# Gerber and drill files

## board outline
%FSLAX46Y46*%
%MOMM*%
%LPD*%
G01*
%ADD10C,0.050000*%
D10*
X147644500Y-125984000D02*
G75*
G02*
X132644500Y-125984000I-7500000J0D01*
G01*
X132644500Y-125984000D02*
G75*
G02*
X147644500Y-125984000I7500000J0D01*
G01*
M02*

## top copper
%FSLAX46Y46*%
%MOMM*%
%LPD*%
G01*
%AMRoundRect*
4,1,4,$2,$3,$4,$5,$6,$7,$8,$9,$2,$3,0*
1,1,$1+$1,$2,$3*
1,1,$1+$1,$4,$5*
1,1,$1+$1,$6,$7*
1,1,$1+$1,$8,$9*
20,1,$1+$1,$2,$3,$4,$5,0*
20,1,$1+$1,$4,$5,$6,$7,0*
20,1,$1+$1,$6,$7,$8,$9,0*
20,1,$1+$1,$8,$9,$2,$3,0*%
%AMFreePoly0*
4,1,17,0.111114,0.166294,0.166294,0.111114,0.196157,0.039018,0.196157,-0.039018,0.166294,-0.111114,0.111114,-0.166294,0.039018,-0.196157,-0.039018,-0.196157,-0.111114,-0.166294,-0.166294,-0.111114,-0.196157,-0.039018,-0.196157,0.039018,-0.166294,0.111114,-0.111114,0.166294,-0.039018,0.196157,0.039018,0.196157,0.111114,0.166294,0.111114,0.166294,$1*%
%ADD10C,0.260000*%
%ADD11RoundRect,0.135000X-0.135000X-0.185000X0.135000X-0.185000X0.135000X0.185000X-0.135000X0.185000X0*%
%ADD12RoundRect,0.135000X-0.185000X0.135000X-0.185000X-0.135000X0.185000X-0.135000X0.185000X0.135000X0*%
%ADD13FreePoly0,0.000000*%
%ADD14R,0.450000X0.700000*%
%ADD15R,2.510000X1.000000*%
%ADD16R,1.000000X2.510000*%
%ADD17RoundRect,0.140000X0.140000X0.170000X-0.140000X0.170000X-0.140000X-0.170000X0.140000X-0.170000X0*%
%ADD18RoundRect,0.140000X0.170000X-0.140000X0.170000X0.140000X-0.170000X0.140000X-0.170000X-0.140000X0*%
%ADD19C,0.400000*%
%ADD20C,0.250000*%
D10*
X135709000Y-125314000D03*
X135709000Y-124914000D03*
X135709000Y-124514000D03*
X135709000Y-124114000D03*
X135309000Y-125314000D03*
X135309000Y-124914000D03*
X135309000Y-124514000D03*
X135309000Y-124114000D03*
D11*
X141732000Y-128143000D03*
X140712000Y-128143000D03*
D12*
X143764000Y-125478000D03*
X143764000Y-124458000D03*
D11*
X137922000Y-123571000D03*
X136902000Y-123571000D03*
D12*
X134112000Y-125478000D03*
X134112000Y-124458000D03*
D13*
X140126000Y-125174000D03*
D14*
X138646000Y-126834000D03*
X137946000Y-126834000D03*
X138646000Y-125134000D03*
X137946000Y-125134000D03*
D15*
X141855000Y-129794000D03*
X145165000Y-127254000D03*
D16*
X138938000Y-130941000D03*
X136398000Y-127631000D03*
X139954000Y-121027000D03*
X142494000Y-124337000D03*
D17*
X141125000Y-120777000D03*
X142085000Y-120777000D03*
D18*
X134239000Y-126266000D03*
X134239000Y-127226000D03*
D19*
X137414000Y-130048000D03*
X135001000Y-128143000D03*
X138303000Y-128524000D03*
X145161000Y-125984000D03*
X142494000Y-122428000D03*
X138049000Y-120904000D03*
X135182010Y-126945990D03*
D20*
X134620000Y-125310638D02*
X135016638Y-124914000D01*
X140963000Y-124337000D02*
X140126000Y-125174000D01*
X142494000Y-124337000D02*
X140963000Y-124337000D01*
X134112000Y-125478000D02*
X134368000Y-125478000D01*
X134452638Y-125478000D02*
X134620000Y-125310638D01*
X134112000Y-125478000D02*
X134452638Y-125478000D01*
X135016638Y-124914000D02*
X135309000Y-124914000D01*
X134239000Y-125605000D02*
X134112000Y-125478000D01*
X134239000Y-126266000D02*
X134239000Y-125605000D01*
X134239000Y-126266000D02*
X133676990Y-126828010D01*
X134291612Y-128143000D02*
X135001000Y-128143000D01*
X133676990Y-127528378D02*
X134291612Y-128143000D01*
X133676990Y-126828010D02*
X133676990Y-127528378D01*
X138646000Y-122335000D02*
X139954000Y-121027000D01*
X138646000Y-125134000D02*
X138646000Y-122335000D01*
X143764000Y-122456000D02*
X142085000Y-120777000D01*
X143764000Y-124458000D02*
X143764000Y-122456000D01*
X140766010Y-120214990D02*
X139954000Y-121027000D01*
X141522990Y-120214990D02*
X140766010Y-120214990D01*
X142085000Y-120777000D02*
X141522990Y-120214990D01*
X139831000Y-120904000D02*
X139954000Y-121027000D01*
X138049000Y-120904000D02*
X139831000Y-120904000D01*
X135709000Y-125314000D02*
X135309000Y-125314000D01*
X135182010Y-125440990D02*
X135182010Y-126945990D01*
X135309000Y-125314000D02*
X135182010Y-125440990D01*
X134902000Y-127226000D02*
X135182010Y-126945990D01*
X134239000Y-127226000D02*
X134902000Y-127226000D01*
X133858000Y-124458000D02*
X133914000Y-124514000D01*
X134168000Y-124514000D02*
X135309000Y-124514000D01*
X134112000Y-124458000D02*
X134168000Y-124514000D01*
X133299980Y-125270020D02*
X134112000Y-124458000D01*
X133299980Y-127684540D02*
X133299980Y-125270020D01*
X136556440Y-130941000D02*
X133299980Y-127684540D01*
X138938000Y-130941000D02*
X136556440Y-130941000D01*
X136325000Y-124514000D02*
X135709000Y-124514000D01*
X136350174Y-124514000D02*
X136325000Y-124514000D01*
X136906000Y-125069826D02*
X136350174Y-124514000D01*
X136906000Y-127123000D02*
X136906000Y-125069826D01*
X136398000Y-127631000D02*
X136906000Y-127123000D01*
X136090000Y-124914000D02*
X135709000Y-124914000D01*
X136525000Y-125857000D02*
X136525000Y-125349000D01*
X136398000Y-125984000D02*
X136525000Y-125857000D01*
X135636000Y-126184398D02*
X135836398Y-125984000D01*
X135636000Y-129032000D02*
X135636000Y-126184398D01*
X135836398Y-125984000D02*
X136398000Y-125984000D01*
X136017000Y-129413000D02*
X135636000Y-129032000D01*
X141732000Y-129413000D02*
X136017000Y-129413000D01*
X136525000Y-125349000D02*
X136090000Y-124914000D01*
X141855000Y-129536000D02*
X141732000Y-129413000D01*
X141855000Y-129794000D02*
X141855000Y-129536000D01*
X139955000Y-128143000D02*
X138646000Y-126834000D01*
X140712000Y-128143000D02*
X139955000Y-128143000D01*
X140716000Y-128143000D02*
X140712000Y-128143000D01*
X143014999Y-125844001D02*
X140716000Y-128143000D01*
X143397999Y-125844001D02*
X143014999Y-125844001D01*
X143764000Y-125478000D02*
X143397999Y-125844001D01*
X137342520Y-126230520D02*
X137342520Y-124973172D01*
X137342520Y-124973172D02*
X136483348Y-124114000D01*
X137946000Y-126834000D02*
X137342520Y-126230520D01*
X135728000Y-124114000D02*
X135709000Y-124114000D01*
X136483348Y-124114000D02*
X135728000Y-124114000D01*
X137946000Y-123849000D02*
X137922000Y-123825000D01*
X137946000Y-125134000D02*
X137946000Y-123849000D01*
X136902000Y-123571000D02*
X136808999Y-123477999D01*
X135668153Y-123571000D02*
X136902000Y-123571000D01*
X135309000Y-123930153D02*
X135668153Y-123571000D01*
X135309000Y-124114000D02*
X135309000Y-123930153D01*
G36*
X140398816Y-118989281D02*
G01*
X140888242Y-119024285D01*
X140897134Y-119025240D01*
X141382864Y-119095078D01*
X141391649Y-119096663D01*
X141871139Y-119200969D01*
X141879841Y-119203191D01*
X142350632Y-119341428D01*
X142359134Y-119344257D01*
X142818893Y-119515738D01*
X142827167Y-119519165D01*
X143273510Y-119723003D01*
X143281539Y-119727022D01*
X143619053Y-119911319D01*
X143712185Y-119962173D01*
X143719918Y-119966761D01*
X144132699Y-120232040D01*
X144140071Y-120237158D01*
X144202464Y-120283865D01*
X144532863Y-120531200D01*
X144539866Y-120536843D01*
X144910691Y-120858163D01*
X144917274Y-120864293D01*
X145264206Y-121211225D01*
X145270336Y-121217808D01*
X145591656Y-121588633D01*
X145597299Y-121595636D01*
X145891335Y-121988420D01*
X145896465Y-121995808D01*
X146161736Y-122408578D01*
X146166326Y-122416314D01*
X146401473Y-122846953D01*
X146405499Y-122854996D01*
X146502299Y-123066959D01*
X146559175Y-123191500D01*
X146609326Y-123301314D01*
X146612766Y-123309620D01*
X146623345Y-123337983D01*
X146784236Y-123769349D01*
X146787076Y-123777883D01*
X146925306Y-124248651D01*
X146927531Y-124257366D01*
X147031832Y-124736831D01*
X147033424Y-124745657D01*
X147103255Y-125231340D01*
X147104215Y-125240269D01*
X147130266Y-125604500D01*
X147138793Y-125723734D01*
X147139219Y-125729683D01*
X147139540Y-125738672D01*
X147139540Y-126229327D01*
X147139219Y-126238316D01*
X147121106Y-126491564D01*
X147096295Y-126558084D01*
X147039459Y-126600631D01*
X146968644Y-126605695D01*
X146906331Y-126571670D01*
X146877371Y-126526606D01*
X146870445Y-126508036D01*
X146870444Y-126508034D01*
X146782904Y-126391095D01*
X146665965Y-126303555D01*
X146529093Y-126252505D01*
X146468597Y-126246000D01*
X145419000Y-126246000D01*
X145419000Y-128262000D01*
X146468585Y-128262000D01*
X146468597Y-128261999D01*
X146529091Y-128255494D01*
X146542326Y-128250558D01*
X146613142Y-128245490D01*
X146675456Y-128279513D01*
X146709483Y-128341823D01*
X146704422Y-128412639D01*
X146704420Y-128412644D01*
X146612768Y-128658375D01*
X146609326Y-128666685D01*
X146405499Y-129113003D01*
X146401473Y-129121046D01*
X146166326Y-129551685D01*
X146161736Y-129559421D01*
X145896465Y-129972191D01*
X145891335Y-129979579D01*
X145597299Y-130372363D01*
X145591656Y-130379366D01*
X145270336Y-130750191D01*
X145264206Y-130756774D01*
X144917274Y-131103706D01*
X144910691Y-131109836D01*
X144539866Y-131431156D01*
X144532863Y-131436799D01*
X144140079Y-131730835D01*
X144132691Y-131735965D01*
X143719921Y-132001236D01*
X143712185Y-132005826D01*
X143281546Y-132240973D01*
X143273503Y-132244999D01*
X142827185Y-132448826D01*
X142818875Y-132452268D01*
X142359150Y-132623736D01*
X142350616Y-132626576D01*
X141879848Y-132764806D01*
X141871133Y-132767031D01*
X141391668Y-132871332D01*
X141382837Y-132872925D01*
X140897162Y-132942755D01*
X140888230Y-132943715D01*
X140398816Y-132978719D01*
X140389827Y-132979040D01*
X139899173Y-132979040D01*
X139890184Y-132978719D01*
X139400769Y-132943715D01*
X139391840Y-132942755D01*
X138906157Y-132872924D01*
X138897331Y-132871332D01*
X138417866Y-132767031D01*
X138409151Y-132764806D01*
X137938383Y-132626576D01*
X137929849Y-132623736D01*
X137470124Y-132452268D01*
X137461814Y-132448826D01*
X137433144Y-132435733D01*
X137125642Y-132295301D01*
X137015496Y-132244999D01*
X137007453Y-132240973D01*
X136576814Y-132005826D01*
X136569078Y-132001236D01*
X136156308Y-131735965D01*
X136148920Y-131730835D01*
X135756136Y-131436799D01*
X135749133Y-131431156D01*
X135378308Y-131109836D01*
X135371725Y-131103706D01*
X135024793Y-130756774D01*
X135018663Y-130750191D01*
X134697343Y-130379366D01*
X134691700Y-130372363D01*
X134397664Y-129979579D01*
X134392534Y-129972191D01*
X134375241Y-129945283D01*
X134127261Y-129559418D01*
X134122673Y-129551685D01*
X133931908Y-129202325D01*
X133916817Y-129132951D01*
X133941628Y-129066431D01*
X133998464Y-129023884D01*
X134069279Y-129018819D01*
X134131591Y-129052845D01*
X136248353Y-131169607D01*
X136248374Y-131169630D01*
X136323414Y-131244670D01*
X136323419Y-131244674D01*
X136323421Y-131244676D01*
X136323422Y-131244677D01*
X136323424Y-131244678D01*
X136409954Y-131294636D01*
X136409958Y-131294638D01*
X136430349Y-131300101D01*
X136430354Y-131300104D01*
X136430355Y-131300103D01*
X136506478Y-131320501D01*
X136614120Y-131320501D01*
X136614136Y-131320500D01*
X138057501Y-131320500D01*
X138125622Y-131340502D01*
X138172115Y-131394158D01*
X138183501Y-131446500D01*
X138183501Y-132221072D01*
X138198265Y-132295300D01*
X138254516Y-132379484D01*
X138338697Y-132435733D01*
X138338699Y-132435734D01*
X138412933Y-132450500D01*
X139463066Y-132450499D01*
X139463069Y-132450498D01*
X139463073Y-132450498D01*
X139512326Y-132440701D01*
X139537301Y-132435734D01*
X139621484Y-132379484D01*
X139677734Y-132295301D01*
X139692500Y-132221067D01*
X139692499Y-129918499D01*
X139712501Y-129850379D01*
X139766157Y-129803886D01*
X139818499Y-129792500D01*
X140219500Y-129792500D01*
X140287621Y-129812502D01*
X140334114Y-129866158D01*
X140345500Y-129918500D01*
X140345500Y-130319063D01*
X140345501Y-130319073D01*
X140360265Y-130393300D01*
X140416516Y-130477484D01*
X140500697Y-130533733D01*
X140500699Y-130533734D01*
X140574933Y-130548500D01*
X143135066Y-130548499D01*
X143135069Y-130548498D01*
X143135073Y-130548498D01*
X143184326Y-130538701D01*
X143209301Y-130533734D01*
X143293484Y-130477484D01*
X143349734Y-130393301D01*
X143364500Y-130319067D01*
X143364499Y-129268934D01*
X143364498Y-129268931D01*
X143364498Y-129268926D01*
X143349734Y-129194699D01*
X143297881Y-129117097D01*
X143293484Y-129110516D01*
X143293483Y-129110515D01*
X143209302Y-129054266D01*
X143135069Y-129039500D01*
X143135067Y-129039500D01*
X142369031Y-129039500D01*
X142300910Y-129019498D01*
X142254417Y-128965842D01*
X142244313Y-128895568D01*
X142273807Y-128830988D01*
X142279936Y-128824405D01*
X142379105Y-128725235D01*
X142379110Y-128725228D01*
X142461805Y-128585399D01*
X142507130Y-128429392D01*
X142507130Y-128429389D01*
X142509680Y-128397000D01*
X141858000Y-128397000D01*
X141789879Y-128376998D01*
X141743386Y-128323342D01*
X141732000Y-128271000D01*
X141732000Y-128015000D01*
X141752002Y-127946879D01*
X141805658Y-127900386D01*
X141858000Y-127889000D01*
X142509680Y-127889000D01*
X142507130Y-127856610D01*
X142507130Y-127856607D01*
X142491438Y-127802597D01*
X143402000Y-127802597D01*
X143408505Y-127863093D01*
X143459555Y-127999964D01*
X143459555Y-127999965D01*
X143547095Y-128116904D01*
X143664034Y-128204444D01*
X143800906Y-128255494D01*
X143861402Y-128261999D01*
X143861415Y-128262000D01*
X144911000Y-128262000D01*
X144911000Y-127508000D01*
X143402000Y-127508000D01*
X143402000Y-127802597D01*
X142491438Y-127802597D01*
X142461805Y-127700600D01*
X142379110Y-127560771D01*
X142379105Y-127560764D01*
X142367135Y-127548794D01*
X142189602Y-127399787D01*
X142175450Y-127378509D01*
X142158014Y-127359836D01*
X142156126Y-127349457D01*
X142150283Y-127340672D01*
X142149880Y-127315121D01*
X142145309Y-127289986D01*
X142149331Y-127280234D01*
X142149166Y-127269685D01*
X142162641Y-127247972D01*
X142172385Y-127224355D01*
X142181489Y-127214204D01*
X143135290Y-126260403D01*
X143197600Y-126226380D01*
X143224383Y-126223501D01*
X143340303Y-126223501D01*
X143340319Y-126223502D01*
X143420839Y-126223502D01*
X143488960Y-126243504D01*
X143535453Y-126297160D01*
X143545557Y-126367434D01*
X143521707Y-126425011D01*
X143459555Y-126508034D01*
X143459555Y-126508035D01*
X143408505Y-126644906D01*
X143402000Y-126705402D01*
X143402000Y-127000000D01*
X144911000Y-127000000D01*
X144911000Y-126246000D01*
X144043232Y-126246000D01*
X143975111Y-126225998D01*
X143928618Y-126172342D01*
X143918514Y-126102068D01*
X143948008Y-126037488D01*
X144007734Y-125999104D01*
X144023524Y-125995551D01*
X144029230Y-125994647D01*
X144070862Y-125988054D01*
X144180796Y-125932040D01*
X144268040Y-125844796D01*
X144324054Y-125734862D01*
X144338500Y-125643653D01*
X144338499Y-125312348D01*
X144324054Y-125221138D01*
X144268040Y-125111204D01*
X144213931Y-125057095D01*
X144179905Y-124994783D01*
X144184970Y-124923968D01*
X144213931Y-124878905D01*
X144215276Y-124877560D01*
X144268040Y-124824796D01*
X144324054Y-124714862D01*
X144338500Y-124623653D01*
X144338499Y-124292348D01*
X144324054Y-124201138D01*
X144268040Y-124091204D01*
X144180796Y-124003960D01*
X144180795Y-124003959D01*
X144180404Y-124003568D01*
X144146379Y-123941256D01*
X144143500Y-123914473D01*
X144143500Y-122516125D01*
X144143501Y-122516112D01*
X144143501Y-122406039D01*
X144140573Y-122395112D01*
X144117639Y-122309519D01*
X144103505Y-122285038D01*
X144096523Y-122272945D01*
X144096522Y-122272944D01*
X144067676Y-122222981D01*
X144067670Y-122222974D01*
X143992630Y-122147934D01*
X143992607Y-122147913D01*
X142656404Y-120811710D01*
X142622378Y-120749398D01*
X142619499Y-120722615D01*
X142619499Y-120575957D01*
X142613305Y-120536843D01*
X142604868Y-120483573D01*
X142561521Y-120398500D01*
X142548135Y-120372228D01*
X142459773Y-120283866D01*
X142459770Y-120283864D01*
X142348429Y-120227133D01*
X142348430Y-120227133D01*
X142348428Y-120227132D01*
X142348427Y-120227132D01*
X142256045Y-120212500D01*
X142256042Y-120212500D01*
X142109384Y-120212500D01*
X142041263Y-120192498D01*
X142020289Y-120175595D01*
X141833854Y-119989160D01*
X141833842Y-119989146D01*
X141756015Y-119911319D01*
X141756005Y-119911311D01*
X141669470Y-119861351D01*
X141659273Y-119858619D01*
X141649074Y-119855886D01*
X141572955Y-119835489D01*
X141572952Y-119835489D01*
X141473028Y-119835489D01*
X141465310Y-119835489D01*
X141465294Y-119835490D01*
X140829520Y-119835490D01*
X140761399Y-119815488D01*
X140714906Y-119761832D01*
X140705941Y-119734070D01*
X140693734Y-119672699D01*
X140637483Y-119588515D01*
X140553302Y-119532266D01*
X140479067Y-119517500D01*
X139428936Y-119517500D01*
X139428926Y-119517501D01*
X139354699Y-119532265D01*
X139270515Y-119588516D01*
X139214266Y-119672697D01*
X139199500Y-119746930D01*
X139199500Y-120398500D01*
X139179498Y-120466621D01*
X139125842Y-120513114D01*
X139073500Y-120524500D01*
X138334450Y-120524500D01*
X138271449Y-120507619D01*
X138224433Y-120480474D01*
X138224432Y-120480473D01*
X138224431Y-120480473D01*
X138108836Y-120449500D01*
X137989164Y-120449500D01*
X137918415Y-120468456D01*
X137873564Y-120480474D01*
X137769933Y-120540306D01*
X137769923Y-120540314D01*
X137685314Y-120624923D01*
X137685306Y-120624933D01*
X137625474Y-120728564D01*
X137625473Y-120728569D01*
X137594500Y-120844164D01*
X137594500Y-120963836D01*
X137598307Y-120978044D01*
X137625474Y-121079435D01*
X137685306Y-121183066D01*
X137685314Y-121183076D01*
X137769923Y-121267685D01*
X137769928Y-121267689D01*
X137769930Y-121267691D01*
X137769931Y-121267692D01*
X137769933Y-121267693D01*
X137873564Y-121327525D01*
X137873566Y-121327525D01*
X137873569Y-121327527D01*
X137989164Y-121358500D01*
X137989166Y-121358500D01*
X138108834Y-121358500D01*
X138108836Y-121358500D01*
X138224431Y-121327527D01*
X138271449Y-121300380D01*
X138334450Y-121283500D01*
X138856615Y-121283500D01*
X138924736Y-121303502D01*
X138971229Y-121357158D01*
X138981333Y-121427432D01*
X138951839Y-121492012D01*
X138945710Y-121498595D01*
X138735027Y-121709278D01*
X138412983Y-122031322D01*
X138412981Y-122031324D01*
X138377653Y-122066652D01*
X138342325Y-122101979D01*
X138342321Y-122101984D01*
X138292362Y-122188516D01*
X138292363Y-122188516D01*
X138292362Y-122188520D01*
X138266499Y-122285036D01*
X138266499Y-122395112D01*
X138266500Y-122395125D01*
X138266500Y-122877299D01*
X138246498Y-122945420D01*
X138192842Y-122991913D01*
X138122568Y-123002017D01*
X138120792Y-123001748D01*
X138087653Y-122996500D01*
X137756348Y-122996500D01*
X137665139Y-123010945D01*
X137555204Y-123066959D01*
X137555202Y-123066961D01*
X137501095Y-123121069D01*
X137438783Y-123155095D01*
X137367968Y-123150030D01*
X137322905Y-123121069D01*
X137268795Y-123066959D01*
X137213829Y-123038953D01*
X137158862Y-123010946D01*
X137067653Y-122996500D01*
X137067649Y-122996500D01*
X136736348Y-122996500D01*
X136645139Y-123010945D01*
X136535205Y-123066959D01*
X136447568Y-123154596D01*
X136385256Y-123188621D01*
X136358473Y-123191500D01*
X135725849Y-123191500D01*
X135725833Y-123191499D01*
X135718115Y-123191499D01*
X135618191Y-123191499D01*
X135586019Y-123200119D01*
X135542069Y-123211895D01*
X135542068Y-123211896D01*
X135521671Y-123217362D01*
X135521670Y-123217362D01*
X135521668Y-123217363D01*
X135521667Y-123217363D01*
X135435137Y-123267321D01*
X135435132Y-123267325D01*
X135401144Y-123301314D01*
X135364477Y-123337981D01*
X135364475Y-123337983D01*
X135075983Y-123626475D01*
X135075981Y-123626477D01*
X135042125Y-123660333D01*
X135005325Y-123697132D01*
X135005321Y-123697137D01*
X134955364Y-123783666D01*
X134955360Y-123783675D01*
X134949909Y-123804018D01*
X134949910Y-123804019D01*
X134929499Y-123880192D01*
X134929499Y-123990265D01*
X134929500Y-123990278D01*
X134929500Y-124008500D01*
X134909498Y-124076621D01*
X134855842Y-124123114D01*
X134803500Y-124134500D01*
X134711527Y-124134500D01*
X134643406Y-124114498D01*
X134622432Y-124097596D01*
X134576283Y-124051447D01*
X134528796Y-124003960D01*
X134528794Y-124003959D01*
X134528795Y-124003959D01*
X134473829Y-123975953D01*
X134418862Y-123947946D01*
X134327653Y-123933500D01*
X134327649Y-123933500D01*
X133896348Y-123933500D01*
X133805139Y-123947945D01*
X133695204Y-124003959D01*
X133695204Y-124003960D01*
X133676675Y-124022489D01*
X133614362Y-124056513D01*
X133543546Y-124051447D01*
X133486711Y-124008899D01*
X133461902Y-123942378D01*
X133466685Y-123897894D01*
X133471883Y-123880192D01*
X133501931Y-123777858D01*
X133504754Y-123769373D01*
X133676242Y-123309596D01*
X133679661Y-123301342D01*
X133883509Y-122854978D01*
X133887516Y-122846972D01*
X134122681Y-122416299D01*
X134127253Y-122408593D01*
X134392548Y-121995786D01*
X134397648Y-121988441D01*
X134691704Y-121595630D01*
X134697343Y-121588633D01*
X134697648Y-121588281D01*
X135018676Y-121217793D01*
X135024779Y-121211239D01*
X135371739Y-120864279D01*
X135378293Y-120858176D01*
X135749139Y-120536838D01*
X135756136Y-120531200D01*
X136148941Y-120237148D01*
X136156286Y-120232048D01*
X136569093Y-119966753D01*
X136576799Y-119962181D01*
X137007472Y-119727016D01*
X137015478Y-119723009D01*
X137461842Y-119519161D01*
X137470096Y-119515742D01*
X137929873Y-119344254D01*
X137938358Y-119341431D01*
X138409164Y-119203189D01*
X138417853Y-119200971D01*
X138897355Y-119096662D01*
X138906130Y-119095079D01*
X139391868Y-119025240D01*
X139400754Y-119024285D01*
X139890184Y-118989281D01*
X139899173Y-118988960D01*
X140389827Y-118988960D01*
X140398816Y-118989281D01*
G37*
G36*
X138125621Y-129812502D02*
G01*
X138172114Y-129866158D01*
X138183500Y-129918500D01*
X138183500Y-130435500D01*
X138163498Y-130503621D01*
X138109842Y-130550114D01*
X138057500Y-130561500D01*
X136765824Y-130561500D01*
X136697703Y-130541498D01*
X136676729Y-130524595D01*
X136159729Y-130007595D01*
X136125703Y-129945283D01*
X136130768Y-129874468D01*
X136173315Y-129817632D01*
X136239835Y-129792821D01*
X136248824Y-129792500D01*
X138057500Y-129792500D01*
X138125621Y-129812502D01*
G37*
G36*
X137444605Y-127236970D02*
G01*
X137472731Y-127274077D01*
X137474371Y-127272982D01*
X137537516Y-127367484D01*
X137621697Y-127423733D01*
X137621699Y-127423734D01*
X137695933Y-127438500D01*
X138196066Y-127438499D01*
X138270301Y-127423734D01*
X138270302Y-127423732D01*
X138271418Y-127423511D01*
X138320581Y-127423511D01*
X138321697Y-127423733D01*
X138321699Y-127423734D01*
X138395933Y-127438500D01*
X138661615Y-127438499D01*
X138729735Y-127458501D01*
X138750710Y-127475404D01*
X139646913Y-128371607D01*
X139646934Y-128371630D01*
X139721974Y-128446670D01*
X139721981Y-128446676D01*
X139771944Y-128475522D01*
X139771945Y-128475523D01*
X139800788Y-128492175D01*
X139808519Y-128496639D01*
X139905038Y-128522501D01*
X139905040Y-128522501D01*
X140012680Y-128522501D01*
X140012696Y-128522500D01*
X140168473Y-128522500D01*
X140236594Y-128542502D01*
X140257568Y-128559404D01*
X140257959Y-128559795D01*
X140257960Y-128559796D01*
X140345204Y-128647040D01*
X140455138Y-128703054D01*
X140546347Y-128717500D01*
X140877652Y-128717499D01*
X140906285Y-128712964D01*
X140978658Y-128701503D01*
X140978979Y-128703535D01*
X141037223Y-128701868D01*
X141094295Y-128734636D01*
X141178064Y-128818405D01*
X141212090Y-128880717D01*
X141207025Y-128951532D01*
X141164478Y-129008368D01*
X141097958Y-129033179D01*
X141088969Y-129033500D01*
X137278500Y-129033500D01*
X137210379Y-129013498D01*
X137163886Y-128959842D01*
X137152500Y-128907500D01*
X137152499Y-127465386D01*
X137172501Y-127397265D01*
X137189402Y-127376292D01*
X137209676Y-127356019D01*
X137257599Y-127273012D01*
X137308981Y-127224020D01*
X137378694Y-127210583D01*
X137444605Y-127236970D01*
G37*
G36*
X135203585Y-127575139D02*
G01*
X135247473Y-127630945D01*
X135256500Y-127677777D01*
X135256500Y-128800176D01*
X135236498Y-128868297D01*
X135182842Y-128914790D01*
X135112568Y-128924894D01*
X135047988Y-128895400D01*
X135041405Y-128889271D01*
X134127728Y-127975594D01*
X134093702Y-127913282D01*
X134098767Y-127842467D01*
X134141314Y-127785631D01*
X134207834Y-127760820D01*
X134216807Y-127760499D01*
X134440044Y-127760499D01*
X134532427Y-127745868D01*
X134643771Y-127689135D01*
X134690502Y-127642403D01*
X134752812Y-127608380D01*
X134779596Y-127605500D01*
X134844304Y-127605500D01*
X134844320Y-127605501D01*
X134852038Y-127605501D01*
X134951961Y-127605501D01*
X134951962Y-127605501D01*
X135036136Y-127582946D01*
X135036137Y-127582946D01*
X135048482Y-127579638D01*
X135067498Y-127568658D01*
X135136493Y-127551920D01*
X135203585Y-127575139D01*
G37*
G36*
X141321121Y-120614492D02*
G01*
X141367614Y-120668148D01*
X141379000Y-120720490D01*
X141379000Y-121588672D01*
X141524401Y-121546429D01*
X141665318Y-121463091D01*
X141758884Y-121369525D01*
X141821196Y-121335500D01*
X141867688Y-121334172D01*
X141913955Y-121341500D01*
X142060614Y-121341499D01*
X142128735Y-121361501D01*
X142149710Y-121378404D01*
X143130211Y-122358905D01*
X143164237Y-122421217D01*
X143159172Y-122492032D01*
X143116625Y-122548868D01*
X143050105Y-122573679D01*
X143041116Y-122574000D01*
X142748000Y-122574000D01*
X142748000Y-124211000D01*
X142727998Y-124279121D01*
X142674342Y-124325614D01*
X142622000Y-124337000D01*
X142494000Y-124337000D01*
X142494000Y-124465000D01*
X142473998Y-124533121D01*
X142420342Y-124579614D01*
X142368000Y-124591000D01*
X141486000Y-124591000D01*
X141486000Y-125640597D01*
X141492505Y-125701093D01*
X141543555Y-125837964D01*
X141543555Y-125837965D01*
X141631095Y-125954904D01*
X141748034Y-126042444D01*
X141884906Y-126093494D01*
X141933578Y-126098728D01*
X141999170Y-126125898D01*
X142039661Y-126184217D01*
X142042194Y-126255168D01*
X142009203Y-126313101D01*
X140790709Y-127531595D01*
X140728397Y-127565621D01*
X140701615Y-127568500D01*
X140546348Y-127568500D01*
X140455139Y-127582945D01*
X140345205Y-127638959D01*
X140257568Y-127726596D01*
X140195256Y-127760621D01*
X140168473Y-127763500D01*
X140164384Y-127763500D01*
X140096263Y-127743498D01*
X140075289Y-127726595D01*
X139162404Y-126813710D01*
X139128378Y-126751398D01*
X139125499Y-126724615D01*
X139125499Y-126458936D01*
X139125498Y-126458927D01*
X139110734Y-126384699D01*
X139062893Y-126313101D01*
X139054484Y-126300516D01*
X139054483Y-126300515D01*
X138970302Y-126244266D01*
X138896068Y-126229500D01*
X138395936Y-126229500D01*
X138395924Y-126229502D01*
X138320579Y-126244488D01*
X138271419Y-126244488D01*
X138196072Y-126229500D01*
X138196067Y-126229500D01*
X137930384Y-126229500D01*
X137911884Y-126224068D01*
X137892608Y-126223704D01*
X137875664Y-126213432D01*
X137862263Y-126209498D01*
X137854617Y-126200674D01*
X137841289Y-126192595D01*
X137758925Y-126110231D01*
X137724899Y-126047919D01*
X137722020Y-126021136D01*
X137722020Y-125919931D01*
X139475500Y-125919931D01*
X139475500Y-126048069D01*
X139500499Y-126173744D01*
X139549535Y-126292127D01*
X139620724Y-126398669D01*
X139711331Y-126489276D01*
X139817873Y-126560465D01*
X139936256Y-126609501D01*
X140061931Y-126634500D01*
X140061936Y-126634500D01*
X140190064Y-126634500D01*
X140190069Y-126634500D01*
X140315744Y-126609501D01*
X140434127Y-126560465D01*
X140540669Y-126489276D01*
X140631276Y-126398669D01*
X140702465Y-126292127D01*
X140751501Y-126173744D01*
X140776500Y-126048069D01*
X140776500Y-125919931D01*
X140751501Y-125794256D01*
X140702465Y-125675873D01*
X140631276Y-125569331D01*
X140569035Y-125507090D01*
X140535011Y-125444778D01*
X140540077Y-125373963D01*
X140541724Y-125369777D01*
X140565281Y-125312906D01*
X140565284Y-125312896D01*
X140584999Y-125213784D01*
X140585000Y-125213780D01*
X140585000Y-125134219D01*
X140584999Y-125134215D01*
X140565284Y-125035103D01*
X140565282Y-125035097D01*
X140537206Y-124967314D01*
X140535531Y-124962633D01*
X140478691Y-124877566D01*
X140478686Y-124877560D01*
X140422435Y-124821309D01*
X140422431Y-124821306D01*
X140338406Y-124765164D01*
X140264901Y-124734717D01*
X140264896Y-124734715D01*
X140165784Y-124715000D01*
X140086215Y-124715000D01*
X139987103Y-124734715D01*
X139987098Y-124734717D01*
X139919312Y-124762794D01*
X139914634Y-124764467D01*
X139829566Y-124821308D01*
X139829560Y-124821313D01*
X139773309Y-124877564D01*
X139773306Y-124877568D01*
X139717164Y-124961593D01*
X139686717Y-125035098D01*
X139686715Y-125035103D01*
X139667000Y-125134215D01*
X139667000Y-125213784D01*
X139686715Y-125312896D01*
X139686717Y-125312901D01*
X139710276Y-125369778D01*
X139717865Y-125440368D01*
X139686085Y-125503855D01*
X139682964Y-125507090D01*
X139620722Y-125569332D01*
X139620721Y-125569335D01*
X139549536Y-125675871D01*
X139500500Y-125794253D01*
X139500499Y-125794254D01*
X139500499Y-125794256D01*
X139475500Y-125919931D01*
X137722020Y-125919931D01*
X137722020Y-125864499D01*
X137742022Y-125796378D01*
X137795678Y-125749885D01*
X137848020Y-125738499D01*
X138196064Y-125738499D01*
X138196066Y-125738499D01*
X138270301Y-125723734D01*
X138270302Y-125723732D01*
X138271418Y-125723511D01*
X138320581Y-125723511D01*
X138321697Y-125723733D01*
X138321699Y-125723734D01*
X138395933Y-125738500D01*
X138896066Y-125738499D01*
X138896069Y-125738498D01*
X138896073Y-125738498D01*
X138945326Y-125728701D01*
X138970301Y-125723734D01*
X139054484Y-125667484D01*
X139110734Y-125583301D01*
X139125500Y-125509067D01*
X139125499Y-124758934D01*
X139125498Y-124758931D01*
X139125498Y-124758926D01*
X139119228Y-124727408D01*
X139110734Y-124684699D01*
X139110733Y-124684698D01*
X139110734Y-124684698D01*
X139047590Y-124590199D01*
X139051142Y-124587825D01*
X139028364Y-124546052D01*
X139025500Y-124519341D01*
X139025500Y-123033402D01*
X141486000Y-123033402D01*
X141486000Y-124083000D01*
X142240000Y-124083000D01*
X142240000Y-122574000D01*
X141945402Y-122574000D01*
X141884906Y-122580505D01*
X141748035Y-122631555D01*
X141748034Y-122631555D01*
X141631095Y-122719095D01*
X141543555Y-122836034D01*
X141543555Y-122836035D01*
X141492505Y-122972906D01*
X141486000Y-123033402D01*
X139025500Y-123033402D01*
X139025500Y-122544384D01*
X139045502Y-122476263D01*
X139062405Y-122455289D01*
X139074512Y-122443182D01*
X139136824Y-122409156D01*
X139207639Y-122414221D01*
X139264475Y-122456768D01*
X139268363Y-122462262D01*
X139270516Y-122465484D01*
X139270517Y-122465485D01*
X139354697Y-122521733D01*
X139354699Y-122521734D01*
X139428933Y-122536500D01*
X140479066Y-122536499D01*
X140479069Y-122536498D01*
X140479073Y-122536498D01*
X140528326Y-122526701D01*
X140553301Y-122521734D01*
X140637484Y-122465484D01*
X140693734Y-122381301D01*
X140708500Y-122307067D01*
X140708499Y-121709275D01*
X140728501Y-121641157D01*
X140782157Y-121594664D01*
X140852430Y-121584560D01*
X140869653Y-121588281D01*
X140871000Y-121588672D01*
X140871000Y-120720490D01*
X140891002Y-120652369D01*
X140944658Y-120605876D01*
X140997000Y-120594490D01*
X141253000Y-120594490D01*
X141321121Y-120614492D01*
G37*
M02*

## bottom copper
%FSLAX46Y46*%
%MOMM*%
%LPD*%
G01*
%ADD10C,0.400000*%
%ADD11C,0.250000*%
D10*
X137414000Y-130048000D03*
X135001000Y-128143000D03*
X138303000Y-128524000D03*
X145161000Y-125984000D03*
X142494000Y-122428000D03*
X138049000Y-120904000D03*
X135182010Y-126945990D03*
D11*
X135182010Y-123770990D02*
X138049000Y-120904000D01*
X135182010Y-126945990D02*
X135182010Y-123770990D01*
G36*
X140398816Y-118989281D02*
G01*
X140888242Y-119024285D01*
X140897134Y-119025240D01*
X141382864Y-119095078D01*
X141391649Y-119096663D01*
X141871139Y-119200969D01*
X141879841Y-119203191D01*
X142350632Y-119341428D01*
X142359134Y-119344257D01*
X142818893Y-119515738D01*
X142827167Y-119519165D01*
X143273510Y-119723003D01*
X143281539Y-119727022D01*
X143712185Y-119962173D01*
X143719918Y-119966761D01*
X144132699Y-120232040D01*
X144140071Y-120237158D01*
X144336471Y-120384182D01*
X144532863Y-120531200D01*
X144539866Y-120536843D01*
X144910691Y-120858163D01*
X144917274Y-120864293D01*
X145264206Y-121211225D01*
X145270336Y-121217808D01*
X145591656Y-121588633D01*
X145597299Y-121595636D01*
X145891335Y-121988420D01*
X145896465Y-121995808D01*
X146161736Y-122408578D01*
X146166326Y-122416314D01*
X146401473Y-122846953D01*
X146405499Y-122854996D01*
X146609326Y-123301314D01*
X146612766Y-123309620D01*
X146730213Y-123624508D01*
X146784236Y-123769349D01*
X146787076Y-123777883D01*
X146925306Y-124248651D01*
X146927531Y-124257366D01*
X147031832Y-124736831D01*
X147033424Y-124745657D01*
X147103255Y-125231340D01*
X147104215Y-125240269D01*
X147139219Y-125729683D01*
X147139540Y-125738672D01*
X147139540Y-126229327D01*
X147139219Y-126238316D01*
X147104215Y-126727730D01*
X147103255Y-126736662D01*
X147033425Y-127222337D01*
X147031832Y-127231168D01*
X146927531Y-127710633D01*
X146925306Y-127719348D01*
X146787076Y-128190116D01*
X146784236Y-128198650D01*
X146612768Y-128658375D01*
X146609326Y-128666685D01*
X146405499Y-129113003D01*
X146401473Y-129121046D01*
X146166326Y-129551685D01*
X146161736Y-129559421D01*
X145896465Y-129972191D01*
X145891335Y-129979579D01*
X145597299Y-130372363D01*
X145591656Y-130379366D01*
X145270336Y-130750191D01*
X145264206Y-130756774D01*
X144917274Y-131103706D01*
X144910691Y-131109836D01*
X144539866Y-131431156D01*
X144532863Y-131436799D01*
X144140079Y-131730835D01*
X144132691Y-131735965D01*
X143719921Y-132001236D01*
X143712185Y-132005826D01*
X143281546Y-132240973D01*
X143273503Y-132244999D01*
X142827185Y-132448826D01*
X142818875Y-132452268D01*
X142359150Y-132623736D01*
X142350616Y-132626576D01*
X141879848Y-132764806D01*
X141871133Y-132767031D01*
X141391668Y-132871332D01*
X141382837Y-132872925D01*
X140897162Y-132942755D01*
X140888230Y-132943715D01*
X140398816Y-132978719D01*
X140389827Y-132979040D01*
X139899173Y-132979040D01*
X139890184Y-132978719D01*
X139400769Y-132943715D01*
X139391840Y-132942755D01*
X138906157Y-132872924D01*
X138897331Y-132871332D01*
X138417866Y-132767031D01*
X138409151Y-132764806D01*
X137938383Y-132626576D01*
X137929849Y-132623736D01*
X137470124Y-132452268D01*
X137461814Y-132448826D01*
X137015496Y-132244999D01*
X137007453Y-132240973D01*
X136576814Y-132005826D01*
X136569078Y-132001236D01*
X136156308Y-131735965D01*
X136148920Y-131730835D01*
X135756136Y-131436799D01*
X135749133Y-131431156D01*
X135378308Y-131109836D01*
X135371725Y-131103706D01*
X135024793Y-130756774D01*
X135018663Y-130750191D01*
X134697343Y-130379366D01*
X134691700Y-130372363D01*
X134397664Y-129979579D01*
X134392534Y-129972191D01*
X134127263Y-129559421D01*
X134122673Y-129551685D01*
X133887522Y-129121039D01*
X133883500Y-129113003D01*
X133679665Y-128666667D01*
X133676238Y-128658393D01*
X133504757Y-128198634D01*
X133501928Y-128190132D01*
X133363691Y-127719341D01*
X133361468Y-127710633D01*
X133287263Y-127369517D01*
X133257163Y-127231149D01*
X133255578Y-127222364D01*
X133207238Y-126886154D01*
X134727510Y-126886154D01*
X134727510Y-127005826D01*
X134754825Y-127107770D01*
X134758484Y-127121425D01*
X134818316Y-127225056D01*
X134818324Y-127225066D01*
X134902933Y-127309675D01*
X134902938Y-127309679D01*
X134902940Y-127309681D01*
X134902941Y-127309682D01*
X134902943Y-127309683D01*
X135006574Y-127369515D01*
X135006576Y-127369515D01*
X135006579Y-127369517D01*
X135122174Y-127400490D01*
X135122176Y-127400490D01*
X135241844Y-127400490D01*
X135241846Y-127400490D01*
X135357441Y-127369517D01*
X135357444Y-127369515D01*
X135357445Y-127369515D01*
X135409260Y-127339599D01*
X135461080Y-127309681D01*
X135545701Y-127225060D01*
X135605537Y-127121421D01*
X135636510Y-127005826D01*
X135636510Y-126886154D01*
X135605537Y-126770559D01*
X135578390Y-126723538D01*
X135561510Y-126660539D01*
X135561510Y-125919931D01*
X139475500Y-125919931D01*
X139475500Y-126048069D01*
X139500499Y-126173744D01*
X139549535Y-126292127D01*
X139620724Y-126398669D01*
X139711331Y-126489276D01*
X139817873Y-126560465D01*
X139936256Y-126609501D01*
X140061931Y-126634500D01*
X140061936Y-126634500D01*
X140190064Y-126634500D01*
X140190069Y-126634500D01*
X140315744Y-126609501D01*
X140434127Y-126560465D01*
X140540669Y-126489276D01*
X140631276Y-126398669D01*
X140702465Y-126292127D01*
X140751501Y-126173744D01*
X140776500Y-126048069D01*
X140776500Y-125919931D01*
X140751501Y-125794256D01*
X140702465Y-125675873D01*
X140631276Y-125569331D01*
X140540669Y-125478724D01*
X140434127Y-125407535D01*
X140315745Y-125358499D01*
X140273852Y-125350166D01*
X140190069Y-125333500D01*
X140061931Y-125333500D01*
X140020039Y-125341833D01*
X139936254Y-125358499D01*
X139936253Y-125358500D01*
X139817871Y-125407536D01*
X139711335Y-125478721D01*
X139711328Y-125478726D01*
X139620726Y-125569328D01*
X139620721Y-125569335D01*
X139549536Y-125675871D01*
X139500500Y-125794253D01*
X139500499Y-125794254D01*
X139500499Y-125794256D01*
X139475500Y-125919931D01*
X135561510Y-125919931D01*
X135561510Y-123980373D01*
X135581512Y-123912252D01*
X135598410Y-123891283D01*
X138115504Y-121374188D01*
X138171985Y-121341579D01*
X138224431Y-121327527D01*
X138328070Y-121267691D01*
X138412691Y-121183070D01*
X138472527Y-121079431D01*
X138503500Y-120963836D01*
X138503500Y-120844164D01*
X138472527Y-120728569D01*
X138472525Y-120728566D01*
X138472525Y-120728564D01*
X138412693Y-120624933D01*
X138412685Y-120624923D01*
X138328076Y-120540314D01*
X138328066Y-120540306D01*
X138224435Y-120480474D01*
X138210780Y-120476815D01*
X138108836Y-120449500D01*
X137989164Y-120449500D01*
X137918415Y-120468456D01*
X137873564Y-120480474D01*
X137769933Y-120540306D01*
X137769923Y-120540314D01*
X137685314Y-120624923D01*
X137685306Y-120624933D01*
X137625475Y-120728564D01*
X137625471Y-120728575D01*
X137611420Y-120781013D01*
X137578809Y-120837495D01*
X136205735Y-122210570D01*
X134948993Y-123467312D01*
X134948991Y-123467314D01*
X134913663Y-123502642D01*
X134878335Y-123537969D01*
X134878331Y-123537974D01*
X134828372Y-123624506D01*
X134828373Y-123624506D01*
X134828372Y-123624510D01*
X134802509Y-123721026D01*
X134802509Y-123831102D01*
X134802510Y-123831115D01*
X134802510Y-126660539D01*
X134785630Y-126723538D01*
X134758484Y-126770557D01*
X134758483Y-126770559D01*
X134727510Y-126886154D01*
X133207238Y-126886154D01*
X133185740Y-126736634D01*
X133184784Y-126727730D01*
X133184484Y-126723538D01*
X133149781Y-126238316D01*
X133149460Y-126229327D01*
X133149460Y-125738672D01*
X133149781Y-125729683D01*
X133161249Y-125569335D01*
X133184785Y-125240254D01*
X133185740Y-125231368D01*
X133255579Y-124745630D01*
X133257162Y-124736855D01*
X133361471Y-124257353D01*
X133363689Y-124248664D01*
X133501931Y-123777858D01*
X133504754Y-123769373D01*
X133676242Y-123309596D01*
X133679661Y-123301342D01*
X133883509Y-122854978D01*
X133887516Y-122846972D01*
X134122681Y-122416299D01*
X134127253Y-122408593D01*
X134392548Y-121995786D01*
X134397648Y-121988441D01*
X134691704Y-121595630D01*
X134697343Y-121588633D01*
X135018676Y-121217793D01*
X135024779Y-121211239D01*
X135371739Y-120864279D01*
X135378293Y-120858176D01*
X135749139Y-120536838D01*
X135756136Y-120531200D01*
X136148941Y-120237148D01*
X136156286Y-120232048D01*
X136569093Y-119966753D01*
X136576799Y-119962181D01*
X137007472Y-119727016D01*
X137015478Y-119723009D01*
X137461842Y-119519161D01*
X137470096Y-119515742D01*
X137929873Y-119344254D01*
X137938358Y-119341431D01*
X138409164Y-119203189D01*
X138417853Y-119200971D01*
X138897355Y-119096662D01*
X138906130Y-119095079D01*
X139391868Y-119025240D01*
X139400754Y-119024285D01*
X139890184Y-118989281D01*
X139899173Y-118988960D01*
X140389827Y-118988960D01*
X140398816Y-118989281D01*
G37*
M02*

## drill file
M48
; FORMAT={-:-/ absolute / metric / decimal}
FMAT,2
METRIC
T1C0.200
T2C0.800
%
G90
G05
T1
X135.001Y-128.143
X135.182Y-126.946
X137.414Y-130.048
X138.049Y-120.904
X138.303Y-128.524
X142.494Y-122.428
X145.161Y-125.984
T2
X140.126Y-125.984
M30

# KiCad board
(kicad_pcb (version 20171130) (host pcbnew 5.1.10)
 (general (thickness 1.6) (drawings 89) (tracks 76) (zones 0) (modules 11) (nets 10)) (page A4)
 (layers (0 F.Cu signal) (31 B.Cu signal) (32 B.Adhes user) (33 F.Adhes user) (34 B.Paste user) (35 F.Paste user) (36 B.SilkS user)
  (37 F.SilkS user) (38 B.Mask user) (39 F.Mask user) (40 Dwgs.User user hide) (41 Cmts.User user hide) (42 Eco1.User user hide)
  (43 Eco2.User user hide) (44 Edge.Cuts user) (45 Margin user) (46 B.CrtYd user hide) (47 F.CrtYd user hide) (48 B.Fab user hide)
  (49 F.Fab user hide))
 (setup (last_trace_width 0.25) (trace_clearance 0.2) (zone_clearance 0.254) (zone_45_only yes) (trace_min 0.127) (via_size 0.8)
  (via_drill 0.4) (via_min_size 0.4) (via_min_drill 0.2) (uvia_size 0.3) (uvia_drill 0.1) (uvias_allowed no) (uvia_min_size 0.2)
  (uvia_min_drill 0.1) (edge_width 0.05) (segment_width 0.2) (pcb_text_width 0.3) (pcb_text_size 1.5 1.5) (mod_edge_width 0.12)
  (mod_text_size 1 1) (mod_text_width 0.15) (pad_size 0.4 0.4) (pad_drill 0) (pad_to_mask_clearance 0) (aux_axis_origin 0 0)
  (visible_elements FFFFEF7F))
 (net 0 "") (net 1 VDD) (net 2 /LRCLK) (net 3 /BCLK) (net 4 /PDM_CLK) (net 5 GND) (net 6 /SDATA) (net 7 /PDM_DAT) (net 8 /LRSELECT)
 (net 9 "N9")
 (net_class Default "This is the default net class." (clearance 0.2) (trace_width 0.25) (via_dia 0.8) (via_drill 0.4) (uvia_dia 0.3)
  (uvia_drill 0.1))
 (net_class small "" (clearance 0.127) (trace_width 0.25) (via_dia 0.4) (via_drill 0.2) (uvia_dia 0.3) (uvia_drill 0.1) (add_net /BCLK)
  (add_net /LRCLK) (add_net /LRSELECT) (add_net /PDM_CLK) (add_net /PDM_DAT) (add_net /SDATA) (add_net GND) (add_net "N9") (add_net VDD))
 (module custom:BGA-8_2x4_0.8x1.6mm (layer F.Cu) (at 135.509 124.714)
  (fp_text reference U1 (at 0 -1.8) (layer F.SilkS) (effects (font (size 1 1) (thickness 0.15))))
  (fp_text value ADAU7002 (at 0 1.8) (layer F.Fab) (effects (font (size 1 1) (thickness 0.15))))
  (pad D2 smd circle (at 0.2 0.6) (size 0.26 0.26) (layers F.Cu F.Paste F.Mask) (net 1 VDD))
  (pad C2 smd circle (at 0.2 0.2) (size 0.26 0.26) (layers F.Cu F.Paste F.Mask) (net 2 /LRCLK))
  (pad B2 smd circle (at 0.2 -0.2) (size 0.26 0.26) (layers F.Cu F.Paste F.Mask) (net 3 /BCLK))
  (pad A2 smd circle (at 0.2 -0.6) (size 0.26 0.26) (layers F.Cu F.Paste F.Mask) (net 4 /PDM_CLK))
  (pad D1 smd circle (at -0.2 0.6) (size 0.26 0.26) (layers F.Cu F.Paste F.Mask) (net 1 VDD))
  (pad C1 smd circle (at -0.2 0.2) (size 0.26 0.26) (layers F.Cu F.Paste F.Mask) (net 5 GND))
  (pad B1 smd circle (at -0.2 -0.2) (size 0.26 0.26) (layers F.Cu F.Paste F.Mask) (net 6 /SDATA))
  (pad A1 smd circle (at -0.2 -0.6) (size 0.26 0.26) (layers F.Cu F.Paste F.Mask) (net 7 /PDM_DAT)))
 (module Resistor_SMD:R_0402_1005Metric (layer F.Cu) (at 141.222 128.143)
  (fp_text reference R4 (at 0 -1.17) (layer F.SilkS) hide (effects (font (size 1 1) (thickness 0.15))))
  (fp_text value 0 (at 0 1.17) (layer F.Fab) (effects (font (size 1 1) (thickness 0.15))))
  (pad 2 smd roundrect (at 0.51 0) (size 0.54 0.64) (layers F.Cu F.Paste F.Mask) (roundrect_rratio 0.25) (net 5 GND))
  (pad 1 smd roundrect (at -0.51 0) (size 0.54 0.64) (layers F.Cu F.Paste F.Mask) (roundrect_rratio 0.25) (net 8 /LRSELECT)))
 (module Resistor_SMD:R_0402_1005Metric (layer F.Cu) (at 143.764 124.968 270)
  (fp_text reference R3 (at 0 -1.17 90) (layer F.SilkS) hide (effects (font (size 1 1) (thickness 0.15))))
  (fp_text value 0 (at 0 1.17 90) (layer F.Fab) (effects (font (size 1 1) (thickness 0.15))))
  (pad 2 smd roundrect (at 0.51 0 270) (size 0.54 0.64) (layers F.Cu F.Paste F.Mask) (roundrect_rratio 0.25) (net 8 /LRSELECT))
  (pad 1 smd roundrect (at -0.51 0 270) (size 0.54 0.64) (layers F.Cu F.Paste F.Mask) (roundrect_rratio 0.25) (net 1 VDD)))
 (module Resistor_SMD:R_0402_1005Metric (layer F.Cu) (at 137.412 123.571)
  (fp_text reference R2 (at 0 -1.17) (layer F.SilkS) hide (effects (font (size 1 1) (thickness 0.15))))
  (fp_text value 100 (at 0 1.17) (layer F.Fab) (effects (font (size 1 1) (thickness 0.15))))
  (pad 2 smd roundrect (at 0.51 0) (size 0.54 0.64) (layers F.Cu F.Paste F.Mask) (roundrect_rratio 0.25) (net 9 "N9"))
  (pad 1 smd roundrect (at -0.51 0) (size 0.54 0.64) (layers F.Cu F.Paste F.Mask) (roundrect_rratio 0.25) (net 7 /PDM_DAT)))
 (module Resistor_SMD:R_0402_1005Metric (layer F.Cu) (at 134.112 124.968 270)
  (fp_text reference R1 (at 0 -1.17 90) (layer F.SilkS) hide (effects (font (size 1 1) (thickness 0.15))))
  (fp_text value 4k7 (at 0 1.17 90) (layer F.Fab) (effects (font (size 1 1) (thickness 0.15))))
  (pad 2 smd roundrect (at 0.51 0 270) (size 0.54 0.64) (layers F.Cu F.Paste F.Mask) (roundrect_rratio 0.25) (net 5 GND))
  (pad 1 smd roundrect (at -0.51 0 270) (size 0.54 0.64) (layers F.Cu F.Paste F.Mask) (roundrect_rratio 0.25) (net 6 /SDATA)))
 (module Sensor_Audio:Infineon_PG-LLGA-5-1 (layer F.Cu) (at 139.446 125.984)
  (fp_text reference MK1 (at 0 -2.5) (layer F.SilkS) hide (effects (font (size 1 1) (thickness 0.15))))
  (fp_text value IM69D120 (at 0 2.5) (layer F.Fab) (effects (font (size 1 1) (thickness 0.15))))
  (pad 5 smd custom (at 0.68 -0.81) (size 0.4 0.4) (layers F.Cu F.Mask) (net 5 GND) (zone_connect 0)
   (options (clearance outline) (anchor circle)) (primitives))
  (pad "" smd custom (at 1.08 -0.693) (size 0.3 0.3) (layers F.Paste) (zone_connect 0) (options (clearance outline) (anchor circle))
   (primitives))
  (pad "" smd custom (at 0.28 -0.693) (size 0.3 0.3) (layers F.Paste) (zone_connect 0) (options (clearance outline) (anchor circle))
   (primitives))
  (pad "" smd custom (at -0.12 0) (size 0.3 0.3) (layers F.Paste) (zone_connect 0) (options (clearance outline) (anchor circle))
   (primitives))
  (pad "" smd custom (at 0.28 0.693) (size 0.3 0.3) (layers F.Paste) (zone_connect 0) (options (clearance outline) (anchor circle))
   (primitives))
  (pad "" smd custom (at 1.08 0.693) (size 0.3 0.3) (layers F.Paste) (zone_connect 0) (options (clearance outline) (anchor circle))
   (primitives))
  (pad "" smd custom (at 1.48 0) (size 0.3 0.3) (layers F.Paste) (zone_connect 0) (options (clearance outline) (anchor circle)) (primitives))
  (pad "" smd custom (at -0.8 0.725) (size 0.3 0.3) (layers F.Paste) (zone_connect 0) (options (clearance outline) (anchor circle))
   (primitives))
  (pad "" smd custom (at -1.5 0.725) (size 0.3 0.3) (layers F.Paste) (zone_connect 0) (options (clearance outline) (anchor circle))
   (primitives))
  (pad "" smd custom (at -0.8 -0.725) (size 0.3 0.3) (layers F.Paste) (zone_connect 0) (options (clearance outline) (anchor circle))
   (primitives))
  (pad "" smd custom (at -1.5 -0.725) (size 0.3 0.3) (layers F.Paste) (zone_connect 0) (options (clearance outline) (anchor circle))
   (primitives))
  (pad "" np_thru_hole circle (at 0.68 0) (size 0.8 0.8) (drill 0.8) (layers *.Cu *.Mask))
  (pad 4 smd rect (at -0.8 0.85) (size 0.45 0.7) (layers F.Cu F.Mask) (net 8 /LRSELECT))
  (pad 3 smd rect (at -1.5 0.85) (size 0.45 0.7) (layers F.Cu F.Mask) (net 4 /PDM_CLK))
  (pad 2 smd rect (at -0.8 -0.85) (size 0.45 0.7) (layers F.Cu F.Mask) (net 1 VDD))
  (pad 1 smd rect (at -1.5 -0.85) (size 0.45 0.7) (layers F.Cu F.Mask) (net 9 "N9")))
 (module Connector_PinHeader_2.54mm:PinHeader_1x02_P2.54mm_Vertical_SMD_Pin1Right (layer F.Cu) (at 143.51 128.524 180)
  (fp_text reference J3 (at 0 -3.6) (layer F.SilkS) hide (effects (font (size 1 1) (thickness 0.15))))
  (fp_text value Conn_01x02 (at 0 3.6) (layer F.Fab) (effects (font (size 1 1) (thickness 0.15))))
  (pad 1 smd rect (at 1.655 -1.27 180) (size 2.51 1) (layers F.Cu F.Paste F.Mask) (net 2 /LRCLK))
  (pad 2 smd rect (at -1.655 1.27 180) (size 2.51 1) (layers F.Cu F.Paste F.Mask) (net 5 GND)))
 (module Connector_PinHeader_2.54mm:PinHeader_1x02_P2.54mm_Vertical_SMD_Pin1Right (layer F.Cu) (at 137.668 129.286 270)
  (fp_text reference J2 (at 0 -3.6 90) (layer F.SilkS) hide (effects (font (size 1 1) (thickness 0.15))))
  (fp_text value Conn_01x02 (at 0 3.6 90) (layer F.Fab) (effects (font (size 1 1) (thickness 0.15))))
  (pad 1 smd rect (at 1.655 -1.27 270) (size 2.51 1) (layers F.Cu F.Paste F.Mask) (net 6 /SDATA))
  (pad 2 smd rect (at -1.655 1.27 270) (size 2.51 1) (layers F.Cu F.Paste F.Mask) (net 3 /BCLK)))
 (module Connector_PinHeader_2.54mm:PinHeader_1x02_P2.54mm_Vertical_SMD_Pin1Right (layer F.Cu) (at 141.224 122.682 90)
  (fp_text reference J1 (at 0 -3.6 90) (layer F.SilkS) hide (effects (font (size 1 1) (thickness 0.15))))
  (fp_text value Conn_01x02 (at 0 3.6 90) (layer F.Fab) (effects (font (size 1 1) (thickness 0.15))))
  (pad 1 smd rect (at 1.655 -1.27 90) (size 2.51 1) (layers F.Cu F.Paste F.Mask) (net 1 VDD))
  (pad 2 smd rect (at -1.655 1.27 90) (size 2.51 1) (layers F.Cu F.Paste F.Mask) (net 5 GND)))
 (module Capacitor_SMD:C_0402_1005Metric (layer F.Cu) (at 141.605 120.777 180)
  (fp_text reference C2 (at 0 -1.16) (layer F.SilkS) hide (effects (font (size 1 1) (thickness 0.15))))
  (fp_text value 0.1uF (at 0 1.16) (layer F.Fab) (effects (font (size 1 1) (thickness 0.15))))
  (pad 2 smd roundrect (at 0.48 0 180) (size 0.56 0.62) (layers F.Cu F.Paste F.Mask) (roundrect_rratio 0.25) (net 5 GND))
  (pad 1 smd roundrect (at -0.48 0 180) (size 0.56 0.62) (layers F.Cu F.Paste F.Mask) (roundrect_rratio 0.25) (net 1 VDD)))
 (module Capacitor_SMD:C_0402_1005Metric (layer F.Cu) (at 134.239 126.746 90)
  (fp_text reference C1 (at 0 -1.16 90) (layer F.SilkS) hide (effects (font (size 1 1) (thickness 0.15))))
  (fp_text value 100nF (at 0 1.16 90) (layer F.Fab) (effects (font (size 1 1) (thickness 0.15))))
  (pad 2 smd roundrect (at 0.48 0 90) (size 0.56 0.62) (layers F.Cu F.Paste F.Mask) (roundrect_rratio 0.25) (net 5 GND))
  (pad 1 smd roundrect (at -0.48 0 90) (size 0.56 0.62) (layers F.Cu F.Paste F.Mask) (roundrect_rratio 0.25) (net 1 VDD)))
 (gr_circle (center 140.1445 125.984) (end 147.6445 125.984) (layer Edge.Cuts) (width 0.05))
 (via (at 137.414 130.048) (size 0.4) (drill 0.2) (layers F.Cu B.Cu) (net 5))
 (via (at 135.001 128.143) (size 0.4) (drill 0.2) (layers F.Cu B.Cu) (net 5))
 (via (at 138.303 128.524) (size 0.4) (drill 0.2) (layers F.Cu B.Cu) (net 5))
 (segment (start 134.62 125.310638) (end 135.016638 124.914) (width 0.25) (layer F.Cu) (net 5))
 (segment (start 140.963 124.337) (end 140.126 125.174) (width 0.25) (layer F.Cu) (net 5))
 (segment (start 142.494 124.337) (end 140.963 124.337) (width 0.25) (layer F.Cu) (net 5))
 (segment (start 134.112 125.478) (end 134.368 125.478) (width 0.25) (layer F.Cu) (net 5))
 (segment (start 134.452638 125.478) (end 134.62 125.310638) (width 0.25) (layer F.Cu) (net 5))
 (segment (start 134.112 125.478) (end 134.452638 125.478) (width 0.25) (layer F.Cu) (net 5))
 (segment (start 135.016638 124.914) (end 135.309 124.914) (width 0.25) (layer F.Cu) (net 5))
 (via (at 145.161 125.984) (size 0.4) (drill 0.2) (layers F.Cu B.Cu) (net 5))
 (via (at 142.494 122.428) (size 0.4) (drill 0.2) (layers F.Cu B.Cu) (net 5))
 (segment (start 134.239 125.605) (end 134.112 125.478) (width 0.25) (layer F.Cu) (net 5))
 (segment (start 134.239 126.266) (end 134.239 125.605) (width 0.25) (layer F.Cu) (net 5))
 (segment (start 134.239 126.266) (end 133.67699 126.82801) (width 0.25) (layer F.Cu) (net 5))
 (segment (start 134.291612 128.143) (end 135.001 128.143) (width 0.25) (layer F.Cu) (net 5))
 (segment (start 133.67699 127.528378) (end 134.291612 128.143) (width 0.25) (layer F.Cu) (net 5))
 (segment (start 133.67699 126.82801) (end 133.67699 127.528378) (width 0.25) (layer F.Cu) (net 5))
 (segment (start 138.646 122.335) (end 139.954 121.027) (width 0.25) (layer F.Cu) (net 1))
 (segment (start 138.646 125.134) (end 138.646 122.335) (width 0.25) (layer F.Cu) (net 1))
 (segment (start 143.764 122.456) (end 142.085 120.777) (width 0.25) (layer F.Cu) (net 1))
 (segment (start 143.764 124.458) (end 143.764 122.456) (width 0.25) (layer F.Cu) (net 1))
 (segment (start 140.76601 120.21499) (end 139.954 121.027) (width 0.25) (layer F.Cu) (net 1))
 (segment (start 141.52299 120.21499) (end 140.76601 120.21499) (width 0.25) (layer F.Cu) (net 1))
 (segment (start 142.085 120.777) (end 141.52299 120.21499) (width 0.25) (layer F.Cu) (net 1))
 (via (at 138.049 120.904) (size 0.4) (drill 0.2) (layers F.Cu B.Cu) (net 1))
 (segment (start 139.831 120.904) (end 139.954 121.027) (width 0.25) (layer F.Cu) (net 1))
 (segment (start 138.049 120.904) (end 139.831 120.904) (width 0.25) (layer F.Cu) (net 1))
 (segment (start 135.709 125.314) (end 135.309 125.314) (width 0.25) (layer F.Cu) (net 1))
 (segment (start 135.18201 125.44099) (end 135.18201 126.94599) (width 0.25) (layer F.Cu) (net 1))
 (segment (start 135.309 125.314) (end 135.18201 125.44099) (width 0.25) (layer F.Cu) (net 1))
 (via (at 135.18201 126.94599) (size 0.4) (drill 0.2) (layers F.Cu B.Cu) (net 1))
 (segment (start 135.18201 123.77099) (end 138.049 120.904) (width 0.25) (layer B.Cu) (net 1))
 (segment (start 135.18201 126.94599) (end 135.18201 123.77099) (width 0.25) (layer B.Cu) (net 1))
 (segment (start 134.902 127.226) (end 135.18201 126.94599) (width 0.25) (layer F.Cu) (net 1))
 (segment (start 134.239 127.226) (end 134.902 127.226) (width 0.25) (layer F.Cu) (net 1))
 (segment (start 133.858 124.458) (end 133.914 124.514) (width 0.25) (layer F.Cu) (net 6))
 (segment (start 134.168 124.514) (end 135.309 124.514) (width 0.25) (layer F.Cu) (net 6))
 (segment (start 134.112 124.458) (end 134.168 124.514) (width 0.25) (layer F.Cu) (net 6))
 (segment (start 133.29998 125.27002) (end 134.112 124.458) (width 0.25) (layer F.Cu) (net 6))
 (segment (start 133.29998 127.68454) (end 133.29998 125.27002) (width 0.25) (layer F.Cu) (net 6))
 (segment (start 136.55644 130.941) (end 133.29998 127.68454) (width 0.25) (layer F.Cu) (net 6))
 (segment (start 138.938 130.941) (end 136.55644 130.941) (width 0.25) (layer F.Cu) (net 6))
 (segment (start 136.325 124.514) (end 135.709 124.514) (width 0.25) (layer F.Cu) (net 3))
 (segment (start 136.350174 124.514) (end 136.325 124.514) (width 0.25) (layer F.Cu) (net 3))
 (segment (start 136.906 125.069826) (end 136.350174 124.514) (width 0.25) (layer F.Cu) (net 3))
 (segment (start 136.906 127.123) (end 136.906 125.069826) (width 0.25) (layer F.Cu) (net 3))
 (segment (start 136.398 127.631) (end 136.906 127.123) (width 0.25) (layer F.Cu) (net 3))
 (segment (start 136.09 124.914) (end 135.709 124.914) (width 0.25) (layer F.Cu) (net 2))
 (segment (start 136.525 125.857) (end 136.525 125.349) (width 0.25) (layer F.Cu) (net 2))
 (segment (start 136.398 125.984) (end 136.525 125.857) (width 0.25) (layer F.Cu) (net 2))
 (segment (start 135.636 126.184398) (end 135.836398 125.984) (width 0.25) (layer F.Cu) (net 2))
 (segment (start 135.636 129.032) (end 135.636 126.184398) (width 0.25) (layer F.Cu) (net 2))
 (segment (start 135.836398 125.984) (end 136.398 125.984) (width 0.25) (layer F.Cu) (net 2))
 (segment (start 136.017 129.413) (end 135.636 129.032) (width 0.25) (layer F.Cu) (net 2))
 (segment (start 141.732 129.413) (end 136.017 129.413) (width 0.25) (layer F.Cu) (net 2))
 (segment (start 136.525 125.349) (end 136.09 124.914) (width 0.25) (layer F.Cu) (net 2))
 (segment (start 141.855 129.536) (end 141.732 129.413) (width 0.25) (layer F.Cu) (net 2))
 (segment (start 141.855 129.794) (end 141.855 129.536) (width 0.25) (layer F.Cu) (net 2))
 (segment (start 139.955 128.143) (end 138.646 126.834) (width 0.25) (layer F.Cu) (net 8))
 (segment (start 140.712 128.143) (end 139.955 128.143) (width 0.25) (layer F.Cu) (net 8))
 (segment (start 140.716 128.143) (end 140.712 128.143) (width 0.25) (layer F.Cu) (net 8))
 (segment (start 143.014999 125.844001) (end 140.716 128.143) (width 0.25) (layer F.Cu) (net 8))
 (segment (start 143.397999 125.844001) (end 143.014999 125.844001) (width 0.25) (layer F.Cu) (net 8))
 (segment (start 143.764 125.478) (end 143.397999 125.844001) (width 0.25) (layer F.Cu) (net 8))
 (segment (start 137.34252 126.23052) (end 137.34252 124.973172) (width 0.25) (layer F.Cu) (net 4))
 (segment (start 137.34252 124.973172) (end 136.483348 124.114) (width 0.25) (layer F.Cu) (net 4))
 (segment (start 137.946 126.834) (end 137.34252 126.23052) (width 0.25) (layer F.Cu) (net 4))
 (segment (start 135.728 124.114) (end 135.709 124.114) (width 0.25) (layer F.Cu) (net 4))
 (segment (start 136.483348 124.114) (end 135.728 124.114) (width 0.25) (layer F.Cu) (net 4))
 (segment (start 137.946 123.849) (end 137.922 123.825) (width 0.25) (layer F.Cu) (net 9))
 (segment (start 137.946 125.134) (end 137.946 123.849) (width 0.25) (layer F.Cu) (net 9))
 (segment (start 136.902 123.571) (end 136.808999 123.477999) (width 0.25) (layer F.Cu) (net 7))
 (segment (start 135.668153 123.571) (end 136.902 123.571) (width 0.25) (layer F.Cu) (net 7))
 (segment (start 135.309 123.930153) (end 135.668153 123.571) (width 0.25) (layer F.Cu) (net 7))
 (segment (start 135.309 124.114) (end 135.309 123.930153) (width 0.25) (layer F.Cu) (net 7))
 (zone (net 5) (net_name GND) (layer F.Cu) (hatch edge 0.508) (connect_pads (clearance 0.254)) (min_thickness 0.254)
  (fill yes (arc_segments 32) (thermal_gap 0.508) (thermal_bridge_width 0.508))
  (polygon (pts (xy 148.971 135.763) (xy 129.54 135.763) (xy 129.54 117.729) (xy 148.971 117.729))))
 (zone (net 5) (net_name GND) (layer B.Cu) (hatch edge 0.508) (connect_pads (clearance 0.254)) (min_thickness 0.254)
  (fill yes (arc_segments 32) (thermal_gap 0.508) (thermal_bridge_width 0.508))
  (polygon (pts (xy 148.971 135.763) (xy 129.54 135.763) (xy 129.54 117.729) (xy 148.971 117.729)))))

